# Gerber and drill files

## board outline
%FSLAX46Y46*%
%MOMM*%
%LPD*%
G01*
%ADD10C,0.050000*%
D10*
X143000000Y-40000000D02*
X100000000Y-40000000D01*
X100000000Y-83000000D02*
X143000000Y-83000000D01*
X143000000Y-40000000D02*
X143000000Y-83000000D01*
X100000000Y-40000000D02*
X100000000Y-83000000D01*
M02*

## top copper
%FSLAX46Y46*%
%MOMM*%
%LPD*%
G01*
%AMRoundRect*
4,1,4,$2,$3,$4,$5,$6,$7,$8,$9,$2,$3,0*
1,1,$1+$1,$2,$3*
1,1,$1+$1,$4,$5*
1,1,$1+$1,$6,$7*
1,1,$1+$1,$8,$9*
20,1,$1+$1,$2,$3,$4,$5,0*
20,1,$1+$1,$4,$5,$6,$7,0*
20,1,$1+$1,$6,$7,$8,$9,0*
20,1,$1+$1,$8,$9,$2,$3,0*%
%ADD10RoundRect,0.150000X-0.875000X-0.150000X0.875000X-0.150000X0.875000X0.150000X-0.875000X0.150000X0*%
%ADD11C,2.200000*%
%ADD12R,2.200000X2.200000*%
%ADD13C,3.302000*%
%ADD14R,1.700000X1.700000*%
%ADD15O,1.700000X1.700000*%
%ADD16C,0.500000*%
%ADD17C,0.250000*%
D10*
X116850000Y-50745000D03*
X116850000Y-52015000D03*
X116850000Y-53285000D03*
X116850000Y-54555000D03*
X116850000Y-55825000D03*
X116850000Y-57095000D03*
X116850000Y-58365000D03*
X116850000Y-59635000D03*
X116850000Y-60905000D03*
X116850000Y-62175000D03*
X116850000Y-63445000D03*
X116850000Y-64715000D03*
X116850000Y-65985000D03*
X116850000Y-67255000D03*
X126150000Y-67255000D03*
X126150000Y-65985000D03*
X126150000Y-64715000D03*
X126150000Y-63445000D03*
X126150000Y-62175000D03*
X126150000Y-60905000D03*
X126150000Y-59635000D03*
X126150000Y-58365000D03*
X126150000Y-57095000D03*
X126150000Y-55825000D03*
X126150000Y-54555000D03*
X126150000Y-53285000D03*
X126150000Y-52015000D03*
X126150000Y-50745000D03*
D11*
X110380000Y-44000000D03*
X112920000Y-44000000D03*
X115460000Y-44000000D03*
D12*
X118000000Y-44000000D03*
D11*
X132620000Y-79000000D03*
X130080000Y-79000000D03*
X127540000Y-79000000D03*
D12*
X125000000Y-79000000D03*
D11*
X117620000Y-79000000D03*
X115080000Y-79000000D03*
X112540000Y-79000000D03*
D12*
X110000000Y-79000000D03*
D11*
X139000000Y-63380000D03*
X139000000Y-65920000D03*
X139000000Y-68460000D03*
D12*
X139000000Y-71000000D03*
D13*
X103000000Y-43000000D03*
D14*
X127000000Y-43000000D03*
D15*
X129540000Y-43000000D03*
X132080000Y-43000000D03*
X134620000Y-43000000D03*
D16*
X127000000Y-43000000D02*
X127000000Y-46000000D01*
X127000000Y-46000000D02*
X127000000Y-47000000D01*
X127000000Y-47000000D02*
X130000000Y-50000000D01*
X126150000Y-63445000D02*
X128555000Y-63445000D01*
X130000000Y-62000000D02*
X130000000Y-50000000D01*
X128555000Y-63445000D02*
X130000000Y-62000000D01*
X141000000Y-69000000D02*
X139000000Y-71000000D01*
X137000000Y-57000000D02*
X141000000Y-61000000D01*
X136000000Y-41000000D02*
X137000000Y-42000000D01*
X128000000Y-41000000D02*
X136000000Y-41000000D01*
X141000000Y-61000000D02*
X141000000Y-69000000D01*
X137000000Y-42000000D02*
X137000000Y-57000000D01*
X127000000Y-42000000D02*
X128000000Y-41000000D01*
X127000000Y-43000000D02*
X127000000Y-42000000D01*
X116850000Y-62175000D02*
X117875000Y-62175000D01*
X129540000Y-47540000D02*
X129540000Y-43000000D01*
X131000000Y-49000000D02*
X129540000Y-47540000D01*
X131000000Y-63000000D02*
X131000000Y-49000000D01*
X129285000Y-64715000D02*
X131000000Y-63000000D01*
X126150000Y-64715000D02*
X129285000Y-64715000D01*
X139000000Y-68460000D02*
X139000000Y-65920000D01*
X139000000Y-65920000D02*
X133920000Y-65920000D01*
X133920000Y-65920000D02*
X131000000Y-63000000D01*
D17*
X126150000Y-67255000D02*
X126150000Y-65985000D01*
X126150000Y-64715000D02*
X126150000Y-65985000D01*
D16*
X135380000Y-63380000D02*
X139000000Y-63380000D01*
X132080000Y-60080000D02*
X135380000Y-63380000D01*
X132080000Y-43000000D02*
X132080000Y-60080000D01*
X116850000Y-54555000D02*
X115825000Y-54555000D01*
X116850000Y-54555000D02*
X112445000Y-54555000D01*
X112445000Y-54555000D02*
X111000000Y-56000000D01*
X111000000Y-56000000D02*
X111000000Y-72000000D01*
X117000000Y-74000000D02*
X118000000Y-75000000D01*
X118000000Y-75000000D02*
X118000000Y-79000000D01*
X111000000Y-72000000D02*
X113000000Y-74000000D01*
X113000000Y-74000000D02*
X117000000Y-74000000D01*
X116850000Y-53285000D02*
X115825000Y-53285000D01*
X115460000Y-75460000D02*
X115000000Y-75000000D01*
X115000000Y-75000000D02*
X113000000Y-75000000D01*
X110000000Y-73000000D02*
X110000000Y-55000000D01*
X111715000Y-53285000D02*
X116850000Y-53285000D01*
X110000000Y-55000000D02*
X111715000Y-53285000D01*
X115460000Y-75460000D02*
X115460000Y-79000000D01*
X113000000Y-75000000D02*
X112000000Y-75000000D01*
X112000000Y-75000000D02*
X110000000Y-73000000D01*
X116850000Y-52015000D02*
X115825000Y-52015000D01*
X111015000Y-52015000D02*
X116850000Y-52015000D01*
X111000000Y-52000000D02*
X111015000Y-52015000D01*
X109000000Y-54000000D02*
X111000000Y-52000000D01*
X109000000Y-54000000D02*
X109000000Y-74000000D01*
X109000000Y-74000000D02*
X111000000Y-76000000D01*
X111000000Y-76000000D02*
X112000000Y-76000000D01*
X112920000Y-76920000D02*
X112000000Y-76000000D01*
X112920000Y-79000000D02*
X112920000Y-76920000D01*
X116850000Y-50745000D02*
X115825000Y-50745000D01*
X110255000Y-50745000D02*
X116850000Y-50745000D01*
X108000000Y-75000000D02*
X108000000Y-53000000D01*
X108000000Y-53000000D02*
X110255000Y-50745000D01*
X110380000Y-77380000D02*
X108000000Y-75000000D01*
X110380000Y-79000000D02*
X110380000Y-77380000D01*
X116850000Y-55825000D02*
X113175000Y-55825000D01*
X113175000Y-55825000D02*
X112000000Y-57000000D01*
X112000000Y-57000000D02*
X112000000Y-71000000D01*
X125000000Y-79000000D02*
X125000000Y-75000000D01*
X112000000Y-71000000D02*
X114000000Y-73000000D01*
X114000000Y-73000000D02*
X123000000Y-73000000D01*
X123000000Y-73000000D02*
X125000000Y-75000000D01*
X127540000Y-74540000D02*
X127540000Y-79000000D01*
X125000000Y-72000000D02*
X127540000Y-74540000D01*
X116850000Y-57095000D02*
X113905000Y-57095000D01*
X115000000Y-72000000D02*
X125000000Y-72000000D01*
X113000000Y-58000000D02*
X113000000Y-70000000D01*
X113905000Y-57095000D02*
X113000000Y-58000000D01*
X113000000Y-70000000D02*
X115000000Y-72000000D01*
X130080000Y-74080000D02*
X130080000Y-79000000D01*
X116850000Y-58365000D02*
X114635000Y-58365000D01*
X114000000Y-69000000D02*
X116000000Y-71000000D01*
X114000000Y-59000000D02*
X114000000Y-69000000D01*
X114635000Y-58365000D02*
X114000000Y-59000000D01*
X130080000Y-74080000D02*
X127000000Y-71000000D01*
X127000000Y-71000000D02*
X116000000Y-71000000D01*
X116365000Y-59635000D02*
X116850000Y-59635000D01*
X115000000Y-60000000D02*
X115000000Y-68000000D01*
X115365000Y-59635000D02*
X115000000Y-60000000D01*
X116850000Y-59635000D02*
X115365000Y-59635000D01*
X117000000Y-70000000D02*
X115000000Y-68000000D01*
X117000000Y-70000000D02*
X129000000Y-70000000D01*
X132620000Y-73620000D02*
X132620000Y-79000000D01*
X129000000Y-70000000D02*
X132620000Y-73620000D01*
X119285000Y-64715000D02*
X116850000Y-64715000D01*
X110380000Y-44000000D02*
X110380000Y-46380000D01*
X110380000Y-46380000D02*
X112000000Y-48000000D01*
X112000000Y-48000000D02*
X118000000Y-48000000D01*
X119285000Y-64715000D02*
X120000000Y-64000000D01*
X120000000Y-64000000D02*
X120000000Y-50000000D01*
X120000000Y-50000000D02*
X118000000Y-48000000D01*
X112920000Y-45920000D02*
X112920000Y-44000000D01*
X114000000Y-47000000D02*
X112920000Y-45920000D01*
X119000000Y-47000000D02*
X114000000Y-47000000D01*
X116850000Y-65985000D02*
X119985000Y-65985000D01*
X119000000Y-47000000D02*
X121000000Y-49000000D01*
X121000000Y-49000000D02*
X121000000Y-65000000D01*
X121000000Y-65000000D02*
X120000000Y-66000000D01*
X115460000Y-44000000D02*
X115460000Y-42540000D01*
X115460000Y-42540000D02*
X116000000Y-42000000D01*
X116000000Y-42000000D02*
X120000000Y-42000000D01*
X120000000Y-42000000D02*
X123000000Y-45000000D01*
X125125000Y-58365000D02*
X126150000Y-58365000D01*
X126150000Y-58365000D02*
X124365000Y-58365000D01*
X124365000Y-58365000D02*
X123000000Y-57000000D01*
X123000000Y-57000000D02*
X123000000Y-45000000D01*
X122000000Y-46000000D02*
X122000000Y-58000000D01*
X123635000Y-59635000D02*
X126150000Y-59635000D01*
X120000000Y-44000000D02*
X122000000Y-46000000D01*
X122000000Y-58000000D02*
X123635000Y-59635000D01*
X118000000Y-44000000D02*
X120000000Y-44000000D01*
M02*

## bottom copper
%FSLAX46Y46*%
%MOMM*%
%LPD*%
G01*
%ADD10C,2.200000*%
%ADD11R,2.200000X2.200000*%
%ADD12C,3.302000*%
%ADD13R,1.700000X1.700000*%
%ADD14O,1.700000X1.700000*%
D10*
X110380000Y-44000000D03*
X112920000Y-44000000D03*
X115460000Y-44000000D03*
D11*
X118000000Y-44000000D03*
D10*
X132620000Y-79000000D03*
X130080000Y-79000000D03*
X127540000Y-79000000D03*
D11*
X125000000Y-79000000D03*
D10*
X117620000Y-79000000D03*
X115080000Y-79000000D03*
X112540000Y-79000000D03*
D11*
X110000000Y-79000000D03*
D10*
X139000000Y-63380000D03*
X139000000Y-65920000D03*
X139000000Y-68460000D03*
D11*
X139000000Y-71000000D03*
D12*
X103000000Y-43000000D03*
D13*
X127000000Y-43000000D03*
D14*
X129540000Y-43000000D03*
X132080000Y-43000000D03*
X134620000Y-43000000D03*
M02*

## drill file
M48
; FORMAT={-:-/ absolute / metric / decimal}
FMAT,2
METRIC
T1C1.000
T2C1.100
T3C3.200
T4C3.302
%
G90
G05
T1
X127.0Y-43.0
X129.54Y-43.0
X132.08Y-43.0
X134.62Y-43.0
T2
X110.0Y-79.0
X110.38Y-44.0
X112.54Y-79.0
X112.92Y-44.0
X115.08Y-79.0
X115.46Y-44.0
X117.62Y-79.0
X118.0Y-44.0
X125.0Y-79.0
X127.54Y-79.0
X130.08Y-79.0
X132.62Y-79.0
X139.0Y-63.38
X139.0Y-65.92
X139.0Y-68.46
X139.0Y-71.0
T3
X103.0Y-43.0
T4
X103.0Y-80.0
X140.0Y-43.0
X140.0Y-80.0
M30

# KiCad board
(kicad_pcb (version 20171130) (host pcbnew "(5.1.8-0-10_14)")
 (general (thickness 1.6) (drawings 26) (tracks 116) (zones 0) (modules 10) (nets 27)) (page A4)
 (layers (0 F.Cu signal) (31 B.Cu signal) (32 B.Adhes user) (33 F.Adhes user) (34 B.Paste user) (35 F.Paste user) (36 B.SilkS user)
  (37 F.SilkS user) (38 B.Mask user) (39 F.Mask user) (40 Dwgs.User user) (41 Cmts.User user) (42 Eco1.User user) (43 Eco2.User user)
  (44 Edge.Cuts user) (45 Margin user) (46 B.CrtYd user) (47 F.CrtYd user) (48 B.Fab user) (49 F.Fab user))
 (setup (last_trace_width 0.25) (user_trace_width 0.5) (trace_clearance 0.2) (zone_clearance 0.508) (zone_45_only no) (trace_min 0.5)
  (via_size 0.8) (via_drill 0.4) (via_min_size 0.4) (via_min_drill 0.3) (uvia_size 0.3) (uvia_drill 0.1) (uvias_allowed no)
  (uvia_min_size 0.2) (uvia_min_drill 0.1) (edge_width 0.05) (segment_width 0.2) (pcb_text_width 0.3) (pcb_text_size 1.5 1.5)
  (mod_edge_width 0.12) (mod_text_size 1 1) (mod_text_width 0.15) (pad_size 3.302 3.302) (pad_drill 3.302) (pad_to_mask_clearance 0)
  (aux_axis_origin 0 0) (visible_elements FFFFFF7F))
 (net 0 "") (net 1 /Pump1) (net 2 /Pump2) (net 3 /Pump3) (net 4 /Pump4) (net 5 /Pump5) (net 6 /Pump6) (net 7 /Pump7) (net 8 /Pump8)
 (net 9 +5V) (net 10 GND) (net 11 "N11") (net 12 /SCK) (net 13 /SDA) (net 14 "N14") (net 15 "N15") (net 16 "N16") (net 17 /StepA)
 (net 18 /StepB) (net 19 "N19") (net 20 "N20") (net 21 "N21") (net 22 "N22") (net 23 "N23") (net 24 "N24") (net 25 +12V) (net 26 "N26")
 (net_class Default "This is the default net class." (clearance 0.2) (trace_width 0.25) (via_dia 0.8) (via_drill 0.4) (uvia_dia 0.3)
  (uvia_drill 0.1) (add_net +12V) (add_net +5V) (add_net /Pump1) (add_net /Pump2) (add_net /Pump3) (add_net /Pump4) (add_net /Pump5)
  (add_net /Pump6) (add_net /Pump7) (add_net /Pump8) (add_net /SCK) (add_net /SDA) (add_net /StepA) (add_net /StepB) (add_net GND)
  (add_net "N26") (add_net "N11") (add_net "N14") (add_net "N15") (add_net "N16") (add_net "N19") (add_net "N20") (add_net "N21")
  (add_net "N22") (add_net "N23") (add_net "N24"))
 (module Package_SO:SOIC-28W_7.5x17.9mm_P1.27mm (layer F.Cu) (at 121.5 59)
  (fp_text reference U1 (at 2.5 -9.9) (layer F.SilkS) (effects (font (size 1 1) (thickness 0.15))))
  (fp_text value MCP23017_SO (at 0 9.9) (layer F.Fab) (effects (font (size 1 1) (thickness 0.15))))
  (pad 1 smd roundrect (at -4.65 -8.255) (size 2.05 0.6) (layers F.Cu F.Paste F.Mask) (roundrect_rratio 0.25) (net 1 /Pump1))
  (pad 2 smd roundrect (at -4.65 -6.985) (size 2.05 0.6) (layers F.Cu F.Paste F.Mask) (roundrect_rratio 0.25) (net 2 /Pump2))
  (pad 3 smd roundrect (at -4.65 -5.715) (size 2.05 0.6) (layers F.Cu F.Paste F.Mask) (roundrect_rratio 0.25) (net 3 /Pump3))
  (pad 4 smd roundrect (at -4.65 -4.445) (size 2.05 0.6) (layers F.Cu F.Paste F.Mask) (roundrect_rratio 0.25) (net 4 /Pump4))
  (pad 5 smd roundrect (at -4.65 -3.175) (size 2.05 0.6) (layers F.Cu F.Paste F.Mask) (roundrect_rratio 0.25) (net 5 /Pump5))
  (pad 6 smd roundrect (at -4.65 -1.905) (size 2.05 0.6) (layers F.Cu F.Paste F.Mask) (roundrect_rratio 0.25) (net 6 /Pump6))
  (pad 7 smd roundrect (at -4.65 -0.635) (size 2.05 0.6) (layers F.Cu F.Paste F.Mask) (roundrect_rratio 0.25) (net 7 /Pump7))
  (pad 8 smd roundrect (at -4.65 0.635) (size 2.05 0.6) (layers F.Cu F.Paste F.Mask) (roundrect_rratio 0.25) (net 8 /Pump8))
  (pad 9 smd roundrect (at -4.65 1.905) (size 2.05 0.6) (layers F.Cu F.Paste F.Mask) (roundrect_rratio 0.25) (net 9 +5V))
  (pad 10 smd roundrect (at -4.65 3.175) (size 2.05 0.6) (layers F.Cu F.Paste F.Mask) (roundrect_rratio 0.25) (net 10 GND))
  (pad 11 smd roundrect (at -4.65 4.445) (size 2.05 0.6) (layers F.Cu F.Paste F.Mask) (roundrect_rratio 0.25) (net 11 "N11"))
  (pad 12 smd roundrect (at -4.65 5.715) (size 2.05 0.6) (layers F.Cu F.Paste F.Mask) (roundrect_rratio 0.25) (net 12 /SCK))
  (pad 13 smd roundrect (at -4.65 6.985) (size 2.05 0.6) (layers F.Cu F.Paste F.Mask) (roundrect_rratio 0.25) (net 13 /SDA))
  (pad 14 smd roundrect (at -4.65 8.255) (size 2.05 0.6) (layers F.Cu F.Paste F.Mask) (roundrect_rratio 0.25) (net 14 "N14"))
  (pad 15 smd roundrect (at 4.65 8.255) (size 2.05 0.6) (layers F.Cu F.Paste F.Mask) (roundrect_rratio 0.25) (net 10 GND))
  (pad 16 smd roundrect (at 4.65 6.985) (size 2.05 0.6) (layers F.Cu F.Paste F.Mask) (roundrect_rratio 0.25) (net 10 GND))
  (pad 17 smd roundrect (at 4.65 5.715) (size 2.05 0.6) (layers F.Cu F.Paste F.Mask) (roundrect_rratio 0.25) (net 10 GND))
  (pad 18 smd roundrect (at 4.65 4.445) (size 2.05 0.6) (layers F.Cu F.Paste F.Mask) (roundrect_rratio 0.25) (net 9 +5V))
  (pad 19 smd roundrect (at 4.65 3.175) (size 2.05 0.6) (layers F.Cu F.Paste F.Mask) (roundrect_rratio 0.25) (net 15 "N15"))
  (pad 20 smd roundrect (at 4.65 1.905) (size 2.05 0.6) (layers F.Cu F.Paste F.Mask) (roundrect_rratio 0.25) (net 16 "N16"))
  (pad 21 smd roundrect (at 4.65 0.635) (size 2.05 0.6) (layers F.Cu F.Paste F.Mask) (roundrect_rratio 0.25) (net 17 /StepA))
  (pad 22 smd roundrect (at 4.65 -0.635) (size 2.05 0.6) (layers F.Cu F.Paste F.Mask) (roundrect_rratio 0.25) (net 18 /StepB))
  (pad 23 smd roundrect (at 4.65 -1.905) (size 2.05 0.6) (layers F.Cu F.Paste F.Mask) (roundrect_rratio 0.25) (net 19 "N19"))
  (pad 24 smd roundrect (at 4.65 -3.175) (size 2.05 0.6) (layers F.Cu F.Paste F.Mask) (roundrect_rratio 0.25) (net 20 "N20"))
  (pad 25 smd roundrect (at 4.65 -4.445) (size 2.05 0.6) (layers F.Cu F.Paste F.Mask) (roundrect_rratio 0.25) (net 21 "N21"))
  (pad 26 smd roundrect (at 4.65 -5.715) (size 2.05 0.6) (layers F.Cu F.Paste F.Mask) (roundrect_rratio 0.25) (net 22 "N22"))
  (pad 27 smd roundrect (at 4.65 -6.985) (size 2.05 0.6) (layers F.Cu F.Paste F.Mask) (roundrect_rratio 0.25) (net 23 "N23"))
  (pad 28 smd roundrect (at 4.65 -8.255) (size 2.05 0.6) (layers F.Cu F.Paste F.Mask) (roundrect_rratio 0.25) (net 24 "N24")))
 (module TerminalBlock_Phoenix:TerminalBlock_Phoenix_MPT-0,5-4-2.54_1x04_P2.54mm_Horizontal (layer F.Cu) (at 118 44 180)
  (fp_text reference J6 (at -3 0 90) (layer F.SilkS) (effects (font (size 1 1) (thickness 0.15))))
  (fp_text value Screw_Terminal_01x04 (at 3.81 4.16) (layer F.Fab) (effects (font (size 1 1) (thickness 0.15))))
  (pad 4 thru_hole circle (at 7.62 0 180) (size 2.2 2.2) (drill 1.1) (layers *.Cu *.Mask) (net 12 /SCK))
  (pad 3 thru_hole circle (at 5.08 0 180) (size 2.2 2.2) (drill 1.1) (layers *.Cu *.Mask) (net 13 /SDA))
  (pad 2 thru_hole circle (at 2.54 0 180) (size 2.2 2.2) (drill 1.1) (layers *.Cu *.Mask) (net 18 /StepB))
  (pad 1 thru_hole rect (at 0 0 180) (size 2.2 2.2) (drill 1.1) (layers *.Cu *.Mask) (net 17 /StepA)))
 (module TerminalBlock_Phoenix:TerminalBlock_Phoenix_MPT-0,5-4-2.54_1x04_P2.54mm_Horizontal (layer F.Cu) (at 125 79)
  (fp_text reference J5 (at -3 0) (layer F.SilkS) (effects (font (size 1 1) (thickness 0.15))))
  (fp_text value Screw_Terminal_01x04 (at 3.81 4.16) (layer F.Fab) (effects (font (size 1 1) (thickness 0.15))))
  (pad 4 thru_hole circle (at 7.62 0) (size 2.2 2.2) (drill 1.1) (layers *.Cu *.Mask) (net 8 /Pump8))
  (pad 3 thru_hole circle (at 5.08 0) (size 2.2 2.2) (drill 1.1) (layers *.Cu *.Mask) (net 7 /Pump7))
  (pad 2 thru_hole circle (at 2.54 0) (size 2.2 2.2) (drill 1.1) (layers *.Cu *.Mask) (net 6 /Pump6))
  (pad 1 thru_hole rect (at 0 0) (size 2.2 2.2) (drill 1.1) (layers *.Cu *.Mask) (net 5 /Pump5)))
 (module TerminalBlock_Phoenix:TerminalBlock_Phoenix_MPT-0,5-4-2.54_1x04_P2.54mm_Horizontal (layer F.Cu) (at 110 79)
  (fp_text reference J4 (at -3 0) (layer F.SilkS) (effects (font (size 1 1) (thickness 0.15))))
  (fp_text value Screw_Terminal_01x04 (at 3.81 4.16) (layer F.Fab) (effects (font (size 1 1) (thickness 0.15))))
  (pad 4 thru_hole circle (at 7.62 0) (size 2.2 2.2) (drill 1.1) (layers *.Cu *.Mask) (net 4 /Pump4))
  (pad 3 thru_hole circle (at 5.08 0) (size 2.2 2.2) (drill 1.1) (layers *.Cu *.Mask) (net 3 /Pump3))
  (pad 2 thru_hole circle (at 2.54 0) (size 2.2 2.2) (drill 1.1) (layers *.Cu *.Mask) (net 2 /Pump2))
  (pad 1 thru_hole rect (at 0 0) (size 2.2 2.2) (drill 1.1) (layers *.Cu *.Mask) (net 1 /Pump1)))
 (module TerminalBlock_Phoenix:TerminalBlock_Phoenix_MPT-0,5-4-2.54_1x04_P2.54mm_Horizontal (layer F.Cu) (at 139 71 90)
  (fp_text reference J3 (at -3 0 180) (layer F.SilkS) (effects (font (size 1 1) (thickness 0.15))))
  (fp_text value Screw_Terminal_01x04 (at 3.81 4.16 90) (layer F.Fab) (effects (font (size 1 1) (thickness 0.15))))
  (pad 4 thru_hole circle (at 7.62 0 90) (size 2.2 2.2) (drill 1.1) (layers *.Cu *.Mask) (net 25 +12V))
  (pad 3 thru_hole circle (at 5.08 0 90) (size 2.2 2.2) (drill 1.1) (layers *.Cu *.Mask) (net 10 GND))
  (pad 2 thru_hole circle (at 2.54 0 90) (size 2.2 2.2) (drill 1.1) (layers *.Cu *.Mask) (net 10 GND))
  (pad 1 thru_hole rect (at 0 0 90) (size 2.2 2.2) (drill 1.1) (layers *.Cu *.Mask) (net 9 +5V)))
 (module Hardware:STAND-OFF (layer F.Cu) (at 140 80)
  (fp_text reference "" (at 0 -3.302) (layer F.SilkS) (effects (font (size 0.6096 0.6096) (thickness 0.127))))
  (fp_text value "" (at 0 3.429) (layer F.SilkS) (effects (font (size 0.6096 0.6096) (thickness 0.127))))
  (pad "" np_thru_hole circle (at 0 0) (size 3.302 3.302) (drill 3.302) (layers *.Cu *.Mask) (solder_mask_margin 0.1016)))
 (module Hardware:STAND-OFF (layer F.Cu) (at 103 80)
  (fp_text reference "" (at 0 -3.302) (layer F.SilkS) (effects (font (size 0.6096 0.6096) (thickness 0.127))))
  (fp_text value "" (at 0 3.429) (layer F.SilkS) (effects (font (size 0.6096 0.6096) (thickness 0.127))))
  (pad "" np_thru_hole circle (at 0 0) (size 3.302 3.302) (drill 3.302) (layers *.Cu *.Mask) (solder_mask_margin 0.1016)))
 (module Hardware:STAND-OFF (layer F.Cu) (at 140 43)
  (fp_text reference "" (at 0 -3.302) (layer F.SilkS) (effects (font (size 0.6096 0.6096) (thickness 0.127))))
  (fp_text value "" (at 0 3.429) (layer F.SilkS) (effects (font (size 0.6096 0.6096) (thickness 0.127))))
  (pad "" np_thru_hole circle (at 0 0) (size 3.302 3.302) (drill 3.302) (layers *.Cu *.Mask) (solder_mask_margin 0.1016)))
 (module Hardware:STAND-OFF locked (layer F.Cu) (at 103 43)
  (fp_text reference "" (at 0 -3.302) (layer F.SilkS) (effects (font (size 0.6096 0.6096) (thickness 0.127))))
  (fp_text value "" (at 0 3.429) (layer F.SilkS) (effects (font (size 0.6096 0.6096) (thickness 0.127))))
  (pad "" np_thru_hole circle (at 0 0) (size 3.302 3.302) (drill 3.2) (layers *.Cu *.Mask) (solder_mask_margin 0.1016)))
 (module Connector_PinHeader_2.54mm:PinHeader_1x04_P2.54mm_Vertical (layer F.Cu) (at 127 43 90)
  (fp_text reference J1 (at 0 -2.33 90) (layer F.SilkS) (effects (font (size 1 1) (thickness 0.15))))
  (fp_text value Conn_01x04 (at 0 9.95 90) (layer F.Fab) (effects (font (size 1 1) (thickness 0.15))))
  (pad 1 thru_hole rect (at 0 0 90) (size 1.7 1.7) (drill 1) (layers *.Cu *.Mask) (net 9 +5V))
  (pad 2 thru_hole oval (at 0 2.54 90) (size 1.7 1.7) (drill 1) (layers *.Cu *.Mask) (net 10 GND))
  (pad 3 thru_hole oval (at 0 5.08 90) (size 1.7 1.7) (drill 1) (layers *.Cu *.Mask) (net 25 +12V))
  (pad 4 thru_hole oval (at 0 7.62 90) (size 1.7 1.7) (drill 1) (layers *.Cu *.Mask) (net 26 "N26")))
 (gr_line (start 143 40) (end 100 40) (layer Edge.Cuts) (width 0.05))
 (gr_line (start 100 83) (end 143 83) (layer Edge.Cuts) (width 0.05))
 (gr_line (start 143 40) (end 143 83) (layer Edge.Cuts) (width 0.05))
 (gr_line (start 100 40) (end 100 83) (layer Edge.Cuts) (width 0.05))
 (segment (start 127 43) (end 127 46) (width 0.5) (layer F.Cu) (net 9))
 (segment (start 127 46) (end 127 47) (width 0.5) (layer F.Cu) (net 9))
 (segment (start 127 47) (end 130 50) (width 0.5) (layer F.Cu) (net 9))
 (segment (start 126.15 63.445) (end 128.555 63.445) (width 0.5) (layer F.Cu) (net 9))
 (segment (start 130 62) (end 130 50) (width 0.5) (layer F.Cu) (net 9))
 (segment (start 128.555 63.445) (end 130 62) (width 0.5) (layer F.Cu) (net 9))
 (segment (start 141 69) (end 139 71) (width 0.5) (layer F.Cu) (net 9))
 (segment (start 137 57) (end 141 61) (width 0.5) (layer F.Cu) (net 9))
 (segment (start 136 41) (end 137 42) (width 0.5) (layer F.Cu) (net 9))
 (segment (start 128 41) (end 136 41) (width 0.5) (layer F.Cu) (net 9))
 (segment (start 141 61) (end 141 69) (width 0.5) (layer F.Cu) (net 9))
 (segment (start 137 42) (end 137 57) (width 0.5) (layer F.Cu) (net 9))
 (segment (start 127 42) (end 128 41) (width 0.5) (layer F.Cu) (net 9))
 (segment (start 127 43) (end 127 42) (width 0.5) (layer F.Cu) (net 9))
 (segment (start 116.85 62.175) (end 117.875 62.175) (width 0.5) (layer F.Cu) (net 10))
 (segment (start 129.54 47.54) (end 129.54 43) (width 0.5) (layer F.Cu) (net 10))
 (segment (start 131 49) (end 129.54 47.54) (width 0.5) (layer F.Cu) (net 10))
 (segment (start 131 63) (end 131 49) (width 0.5) (layer F.Cu) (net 10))
 (segment (start 129.285 64.715) (end 131 63) (width 0.5) (layer F.Cu) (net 10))
 (segment (start 126.15 64.715) (end 129.285 64.715) (width 0.5) (layer F.Cu) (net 10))
 (segment (start 139 68.46) (end 139 65.92) (width 0.5) (layer F.Cu) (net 10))
 (segment (start 139 65.92) (end 133.92 65.92) (width 0.5) (layer F.Cu) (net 10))
 (segment (start 133.92 65.92) (end 131 63) (width 0.5) (layer F.Cu) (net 10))
 (segment (start 126.15 67.255) (end 126.15 65.985) (width 0.25) (layer F.Cu) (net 10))
 (segment (start 126.15 64.715) (end 126.15 65.985) (width 0.25) (layer F.Cu) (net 10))
 (segment (start 135.38 63.38) (end 139 63.38) (width 0.5) (layer F.Cu) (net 25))
 (segment (start 132.08 60.08) (end 135.38 63.38) (width 0.5) (layer F.Cu) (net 25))
 (segment (start 132.08 43) (end 132.08 60.08) (width 0.5) (layer F.Cu) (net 25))
 (segment (start 116.85 54.555) (end 115.825 54.555) (width 0.5) (layer F.Cu) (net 4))
 (segment (start 116.85 54.555) (end 112.445 54.555) (width 0.5) (layer F.Cu) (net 4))
 (segment (start 112.445 54.555) (end 111 56) (width 0.5) (layer F.Cu) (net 4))
 (segment (start 111 56) (end 111 72) (width 0.5) (layer F.Cu) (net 4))
 (segment (start 117 74) (end 118 75) (width 0.5) (layer F.Cu) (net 4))
 (segment (start 118 75) (end 118 79) (width 0.5) (layer F.Cu) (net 4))
 (segment (start 111 72) (end 113 74) (width 0.5) (layer F.Cu) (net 4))
 (segment (start 113 74) (end 117 74) (width 0.5) (layer F.Cu) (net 4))
 (segment (start 116.85 53.285) (end 115.825 53.285) (width 0.5) (layer F.Cu) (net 3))
 (segment (start 115.46 75.46) (end 115 75) (width 0.5) (layer F.Cu) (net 3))
 (segment (start 115 75) (end 113 75) (width 0.5) (layer F.Cu) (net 3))
 (segment (start 110 73) (end 110 55) (width 0.5) (layer F.Cu) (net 3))
 (segment (start 111.715 53.285) (end 116.85 53.285) (width 0.5) (layer F.Cu) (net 3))
 (segment (start 110 55) (end 111.715 53.285) (width 0.5) (layer F.Cu) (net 3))
 (segment (start 115.46 75.46) (end 115.46 79) (width 0.5) (layer F.Cu) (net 3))
 (segment (start 113 75) (end 112 75) (width 0.5) (layer F.Cu) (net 3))
 (segment (start 112 75) (end 110 73) (width 0.5) (layer F.Cu) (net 3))
 (segment (start 116.85 52.015) (end 115.825 52.015) (width 0.5) (layer F.Cu) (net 2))
 (segment (start 111.015 52.015) (end 116.85 52.015) (width 0.5) (layer F.Cu) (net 2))
 (segment (start 111 52) (end 111.015 52.015) (width 0.5) (layer F.Cu) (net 2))
 (segment (start 109 54) (end 111 52) (width 0.5) (layer F.Cu) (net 2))
 (segment (start 109 54) (end 109 74) (width 0.5) (layer F.Cu) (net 2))
 (segment (start 109 74) (end 111 76) (width 0.5) (layer F.Cu) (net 2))
 (segment (start 111 76) (end 112 76) (width 0.5) (layer F.Cu) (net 2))
 (segment (start 112.92 76.92) (end 112 76) (width 0.5) (layer F.Cu) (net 2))
 (segment (start 112.92 79) (end 112.92 76.92) (width 0.5) (layer F.Cu) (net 2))
 (segment (start 116.85 50.745) (end 115.825 50.745) (width 0.5) (layer F.Cu) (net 1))
 (segment (start 110.255 50.745) (end 116.85 50.745) (width 0.5) (layer F.Cu) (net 1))
 (segment (start 108 75) (end 108 53) (width 0.5) (layer F.Cu) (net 1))
 (segment (start 108 53) (end 110.255 50.745) (width 0.5) (layer F.Cu) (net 1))
 (segment (start 110.38 77.38) (end 108 75) (width 0.5) (layer F.Cu) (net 1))
 (segment (start 110.38 79) (end 110.38 77.38) (width 0.5) (layer F.Cu) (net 1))
 (segment (start 116.85 55.825) (end 113.175 55.825) (width 0.5) (layer F.Cu) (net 5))
 (segment (start 113.175 55.825) (end 112 57) (width 0.5) (layer F.Cu) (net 5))
 (segment (start 112 57) (end 112 71) (width 0.5) (layer F.Cu) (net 5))
 (segment (start 125 79) (end 125 75) (width 0.5) (layer F.Cu) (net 5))
 (segment (start 112 71) (end 114 73) (width 0.5) (layer F.Cu) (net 5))
 (segment (start 114 73) (end 123 73) (width 0.5) (layer F.Cu) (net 5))
 (segment (start 123 73) (end 125 75) (width 0.5) (layer F.Cu) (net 5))
 (segment (start 127.54 74.54) (end 127.54 79) (width 0.5) (layer F.Cu) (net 6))
 (segment (start 125 72) (end 127.54 74.54) (width 0.5) (layer F.Cu) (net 6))
 (segment (start 116.85 57.095) (end 113.905 57.095) (width 0.5) (layer F.Cu) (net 6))
 (segment (start 115 72) (end 125 72) (width 0.5) (layer F.Cu) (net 6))
 (segment (start 113 58) (end 113 70) (width 0.5) (layer F.Cu) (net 6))
 (segment (start 113.905 57.095) (end 113 58) (width 0.5) (layer F.Cu) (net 6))
 (segment (start 113 70) (end 115 72) (width 0.5) (layer F.Cu) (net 6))
 (segment (start 130.08 74.08) (end 130.08 79) (width 0.5) (layer F.Cu) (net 7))
 (segment (start 116.85 58.365) (end 114.635 58.365) (width 0.5) (layer F.Cu) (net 7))
 (segment (start 114 69) (end 116 71) (width 0.5) (layer F.Cu) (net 7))
 (segment (start 114 59) (end 114 69) (width 0.5) (layer F.Cu) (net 7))
 (segment (start 114.635 58.365) (end 114 59) (width 0.5) (layer F.Cu) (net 7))
 (segment (start 130.08 74.08) (end 127 71) (width 0.5) (layer F.Cu) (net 7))
 (segment (start 127 71) (end 116 71) (width 0.5) (layer F.Cu) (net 7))
 (segment (start 116.365 59.635) (end 116.85 59.635) (width 0.5) (layer F.Cu) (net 8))
 (segment (start 115 60) (end 115 68) (width 0.5) (layer F.Cu) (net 8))
 (segment (start 115.365 59.635) (end 115 60) (width 0.5) (layer F.Cu) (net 8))
 (segment (start 116.85 59.635) (end 115.365 59.635) (width 0.5) (layer F.Cu) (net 8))
 (segment (start 117 70) (end 115 68) (width 0.5) (layer F.Cu) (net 8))
 (segment (start 117 70) (end 129 70) (width 0.5) (layer F.Cu) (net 8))
 (segment (start 132.62 73.62) (end 132.62 79) (width 0.5) (layer F.Cu) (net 8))
 (segment (start 129 70) (end 132.62 73.62) (width 0.5) (layer F.Cu) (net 8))
 (segment (start 119.285 64.715) (end 116.85 64.715) (width 0.5) (layer F.Cu) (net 12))
 (segment (start 110.38 44) (end 110.38 46.38) (width 0.5) (layer F.Cu) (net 12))
 (segment (start 110.38 46.38) (end 112 48) (width 0.5) (layer F.Cu) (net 12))
 (segment (start 112 48) (end 118 48) (width 0.5) (layer F.Cu) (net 12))
 (segment (start 119.285 64.715) (end 120 64) (width 0.5) (layer F.Cu) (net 12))
 (segment (start 120 64) (end 120 50) (width 0.5) (layer F.Cu) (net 12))
 (segment (start 120 50) (end 118 48) (width 0.5) (layer F.Cu) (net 12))
 (segment (start 112.92 45.92) (end 112.92 44) (width 0.5) (layer F.Cu) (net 13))
 (segment (start 114 47) (end 112.92 45.92) (width 0.5) (layer F.Cu) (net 13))
 (segment (start 119 47) (end 114 47) (width 0.5) (layer F.Cu) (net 13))
 (segment (start 116.85 65.985) (end 119.985 65.985) (width 0.5) (layer F.Cu) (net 13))
 (segment (start 119 47) (end 121 49) (width 0.5) (layer F.Cu) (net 13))
 (segment (start 121 49) (end 121 65) (width 0.5) (layer F.Cu) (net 13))
 (segment (start 121 65) (end 120 66) (width 0.5) (layer F.Cu) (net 13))
 (segment (start 115.46 44) (end 115.46 42.54) (width 0.5) (layer F.Cu) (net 18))
 (segment (start 115.46 42.54) (end 116 42) (width 0.5) (layer F.Cu) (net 18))
 (segment (start 116 42) (end 120 42) (width 0.5) (layer F.Cu) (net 18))
 (segment (start 120 42) (end 123 45) (width 0.5) (layer F.Cu) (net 18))
 (segment (start 125.125 58.365) (end 126.15 58.365) (width 0.5) (layer F.Cu) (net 18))
 (segment (start 126.15 58.365) (end 124.365 58.365) (width 0.5) (layer F.Cu) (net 18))
 (segment (start 124.365 58.365) (end 123 57) (width 0.5) (layer F.Cu) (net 18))
 (segment (start 123 57) (end 123 45) (width 0.5) (layer F.Cu) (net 18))
 (segment (start 122 46) (end 122 58) (width 0.5) (layer F.Cu) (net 17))
 (segment (start 123.635 59.635) (end 126.15 59.635) (width 0.5) (layer F.Cu) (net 17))
 (segment (start 120 44) (end 122 46) (width 0.5) (layer F.Cu) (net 17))
 (segment (start 122 58) (end 123.635 59.635) (width 0.5) (layer F.Cu) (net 17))
 (segment (start 118 44) (end 120 44) (width 0.5) (layer F.Cu) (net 17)))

